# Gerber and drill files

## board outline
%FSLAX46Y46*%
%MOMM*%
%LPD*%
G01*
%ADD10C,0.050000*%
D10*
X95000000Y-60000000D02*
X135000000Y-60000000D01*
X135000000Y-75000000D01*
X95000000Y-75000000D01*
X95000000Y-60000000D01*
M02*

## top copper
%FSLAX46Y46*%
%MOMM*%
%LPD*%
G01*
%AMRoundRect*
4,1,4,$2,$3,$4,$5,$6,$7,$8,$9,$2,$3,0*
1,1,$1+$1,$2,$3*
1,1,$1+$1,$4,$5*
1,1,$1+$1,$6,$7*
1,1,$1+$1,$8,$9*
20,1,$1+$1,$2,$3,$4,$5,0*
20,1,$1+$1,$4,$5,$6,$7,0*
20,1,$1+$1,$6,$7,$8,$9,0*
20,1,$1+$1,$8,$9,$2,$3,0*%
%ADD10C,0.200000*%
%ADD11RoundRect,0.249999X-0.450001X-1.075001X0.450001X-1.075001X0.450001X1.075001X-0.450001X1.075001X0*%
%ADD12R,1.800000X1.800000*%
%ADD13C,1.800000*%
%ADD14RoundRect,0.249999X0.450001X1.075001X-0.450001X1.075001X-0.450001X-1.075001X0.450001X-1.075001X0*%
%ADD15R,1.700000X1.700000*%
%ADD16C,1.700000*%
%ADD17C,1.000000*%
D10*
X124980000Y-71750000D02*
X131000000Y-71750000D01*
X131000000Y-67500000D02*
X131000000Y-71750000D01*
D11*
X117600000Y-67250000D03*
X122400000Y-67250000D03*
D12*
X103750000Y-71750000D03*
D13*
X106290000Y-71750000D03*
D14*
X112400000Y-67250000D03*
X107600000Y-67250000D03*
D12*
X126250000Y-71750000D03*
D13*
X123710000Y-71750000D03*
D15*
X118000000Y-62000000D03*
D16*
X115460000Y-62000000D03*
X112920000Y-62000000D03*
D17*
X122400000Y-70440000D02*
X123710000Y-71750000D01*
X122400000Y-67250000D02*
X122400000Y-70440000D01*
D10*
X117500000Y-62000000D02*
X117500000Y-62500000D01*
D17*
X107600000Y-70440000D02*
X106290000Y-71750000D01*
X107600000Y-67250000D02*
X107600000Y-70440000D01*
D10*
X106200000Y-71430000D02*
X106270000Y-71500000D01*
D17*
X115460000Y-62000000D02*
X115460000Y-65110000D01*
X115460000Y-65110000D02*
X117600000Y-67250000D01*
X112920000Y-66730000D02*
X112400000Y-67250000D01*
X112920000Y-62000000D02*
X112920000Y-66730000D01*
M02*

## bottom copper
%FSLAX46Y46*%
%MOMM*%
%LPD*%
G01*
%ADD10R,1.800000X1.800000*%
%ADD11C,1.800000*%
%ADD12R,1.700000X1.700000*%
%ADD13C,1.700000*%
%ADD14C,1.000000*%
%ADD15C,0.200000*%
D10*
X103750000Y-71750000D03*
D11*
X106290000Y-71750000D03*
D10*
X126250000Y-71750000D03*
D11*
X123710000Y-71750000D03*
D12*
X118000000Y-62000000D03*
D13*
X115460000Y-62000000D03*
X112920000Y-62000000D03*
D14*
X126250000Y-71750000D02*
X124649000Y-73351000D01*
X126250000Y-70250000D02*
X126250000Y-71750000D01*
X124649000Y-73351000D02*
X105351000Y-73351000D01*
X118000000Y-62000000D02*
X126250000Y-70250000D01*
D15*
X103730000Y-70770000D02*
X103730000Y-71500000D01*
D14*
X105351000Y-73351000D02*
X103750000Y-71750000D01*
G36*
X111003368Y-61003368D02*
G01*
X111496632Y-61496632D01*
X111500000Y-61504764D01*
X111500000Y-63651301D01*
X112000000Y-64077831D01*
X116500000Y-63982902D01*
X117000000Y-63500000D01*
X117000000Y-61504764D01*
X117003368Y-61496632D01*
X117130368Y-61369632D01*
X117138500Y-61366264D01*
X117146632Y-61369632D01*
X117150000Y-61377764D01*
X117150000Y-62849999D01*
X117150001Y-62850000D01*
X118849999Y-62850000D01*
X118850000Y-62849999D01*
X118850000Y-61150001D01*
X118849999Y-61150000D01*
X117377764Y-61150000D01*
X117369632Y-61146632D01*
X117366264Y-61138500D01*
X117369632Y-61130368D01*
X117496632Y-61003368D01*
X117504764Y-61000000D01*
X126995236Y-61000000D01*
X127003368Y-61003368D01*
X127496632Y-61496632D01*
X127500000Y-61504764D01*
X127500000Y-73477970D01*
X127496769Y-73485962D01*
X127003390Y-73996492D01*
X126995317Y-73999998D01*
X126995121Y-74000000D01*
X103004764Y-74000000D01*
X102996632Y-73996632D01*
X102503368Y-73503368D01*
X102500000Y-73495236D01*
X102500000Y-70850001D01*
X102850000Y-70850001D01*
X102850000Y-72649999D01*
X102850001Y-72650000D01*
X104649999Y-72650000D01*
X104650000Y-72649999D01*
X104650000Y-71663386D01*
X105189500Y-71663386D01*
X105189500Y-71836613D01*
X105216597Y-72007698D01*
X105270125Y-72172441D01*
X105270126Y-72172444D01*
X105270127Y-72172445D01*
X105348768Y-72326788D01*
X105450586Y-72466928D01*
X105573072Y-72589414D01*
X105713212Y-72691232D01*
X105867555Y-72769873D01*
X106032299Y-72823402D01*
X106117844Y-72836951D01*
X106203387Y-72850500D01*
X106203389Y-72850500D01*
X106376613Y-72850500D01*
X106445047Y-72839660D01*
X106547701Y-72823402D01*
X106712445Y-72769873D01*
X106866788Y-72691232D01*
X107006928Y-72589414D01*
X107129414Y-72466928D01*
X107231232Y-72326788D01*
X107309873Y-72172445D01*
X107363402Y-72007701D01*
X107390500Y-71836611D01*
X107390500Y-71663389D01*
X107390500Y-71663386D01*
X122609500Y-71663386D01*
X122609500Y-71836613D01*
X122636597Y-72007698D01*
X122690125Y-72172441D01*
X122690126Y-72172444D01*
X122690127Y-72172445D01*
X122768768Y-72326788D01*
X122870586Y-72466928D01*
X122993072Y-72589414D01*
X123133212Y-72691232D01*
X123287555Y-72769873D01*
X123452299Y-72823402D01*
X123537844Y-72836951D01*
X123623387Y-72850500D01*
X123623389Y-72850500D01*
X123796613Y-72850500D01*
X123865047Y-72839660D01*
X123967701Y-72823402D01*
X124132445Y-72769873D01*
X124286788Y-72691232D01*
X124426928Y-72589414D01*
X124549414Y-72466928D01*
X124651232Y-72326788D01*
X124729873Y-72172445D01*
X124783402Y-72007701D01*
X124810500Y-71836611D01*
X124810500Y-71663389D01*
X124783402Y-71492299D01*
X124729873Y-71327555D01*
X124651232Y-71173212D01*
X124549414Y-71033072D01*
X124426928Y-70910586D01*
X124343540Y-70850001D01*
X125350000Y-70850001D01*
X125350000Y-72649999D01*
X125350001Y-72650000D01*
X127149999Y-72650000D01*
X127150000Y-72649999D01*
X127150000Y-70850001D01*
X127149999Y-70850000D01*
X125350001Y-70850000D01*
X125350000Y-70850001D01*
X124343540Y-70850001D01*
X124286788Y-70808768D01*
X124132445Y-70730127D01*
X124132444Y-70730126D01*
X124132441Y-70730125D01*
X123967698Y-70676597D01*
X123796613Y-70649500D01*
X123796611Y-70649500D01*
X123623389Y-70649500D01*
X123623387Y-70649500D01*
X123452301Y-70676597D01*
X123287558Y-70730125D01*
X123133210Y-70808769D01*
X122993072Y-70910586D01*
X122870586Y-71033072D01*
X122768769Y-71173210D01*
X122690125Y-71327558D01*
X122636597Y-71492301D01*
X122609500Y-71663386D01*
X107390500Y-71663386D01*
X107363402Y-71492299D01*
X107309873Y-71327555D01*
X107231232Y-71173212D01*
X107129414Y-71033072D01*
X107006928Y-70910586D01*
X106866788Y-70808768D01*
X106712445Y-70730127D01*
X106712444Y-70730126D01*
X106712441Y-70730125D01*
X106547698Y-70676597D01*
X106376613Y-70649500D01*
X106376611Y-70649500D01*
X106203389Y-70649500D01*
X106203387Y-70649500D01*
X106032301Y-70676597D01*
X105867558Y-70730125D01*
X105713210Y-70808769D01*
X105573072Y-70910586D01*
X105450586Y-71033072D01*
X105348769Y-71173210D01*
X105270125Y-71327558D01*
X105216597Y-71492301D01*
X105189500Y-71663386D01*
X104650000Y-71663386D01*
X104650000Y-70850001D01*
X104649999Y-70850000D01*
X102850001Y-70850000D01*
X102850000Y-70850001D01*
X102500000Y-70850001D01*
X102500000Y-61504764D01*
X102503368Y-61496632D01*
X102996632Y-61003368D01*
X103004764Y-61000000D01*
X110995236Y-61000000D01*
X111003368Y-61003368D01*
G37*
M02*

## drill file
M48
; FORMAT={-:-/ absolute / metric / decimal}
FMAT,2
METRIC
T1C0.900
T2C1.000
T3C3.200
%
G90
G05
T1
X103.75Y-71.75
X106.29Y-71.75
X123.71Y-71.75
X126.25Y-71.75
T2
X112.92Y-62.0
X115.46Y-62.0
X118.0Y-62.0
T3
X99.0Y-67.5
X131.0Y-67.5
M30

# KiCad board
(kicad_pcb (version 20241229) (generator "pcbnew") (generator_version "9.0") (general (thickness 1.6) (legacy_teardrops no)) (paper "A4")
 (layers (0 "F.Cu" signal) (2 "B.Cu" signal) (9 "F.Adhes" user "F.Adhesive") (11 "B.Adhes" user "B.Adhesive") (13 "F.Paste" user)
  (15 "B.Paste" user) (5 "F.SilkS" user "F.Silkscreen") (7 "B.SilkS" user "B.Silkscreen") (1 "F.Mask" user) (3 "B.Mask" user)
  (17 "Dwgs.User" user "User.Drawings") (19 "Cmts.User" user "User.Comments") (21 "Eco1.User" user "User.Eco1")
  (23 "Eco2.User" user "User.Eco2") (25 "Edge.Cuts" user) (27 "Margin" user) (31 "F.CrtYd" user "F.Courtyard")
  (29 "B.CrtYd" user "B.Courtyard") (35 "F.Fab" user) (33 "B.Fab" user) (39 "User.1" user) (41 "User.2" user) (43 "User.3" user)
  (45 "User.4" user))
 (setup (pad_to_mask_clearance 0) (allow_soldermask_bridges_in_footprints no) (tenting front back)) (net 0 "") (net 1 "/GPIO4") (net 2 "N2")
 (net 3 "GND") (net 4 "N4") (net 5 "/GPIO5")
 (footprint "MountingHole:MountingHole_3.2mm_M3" (layer "F.Cu") (at 131 67.5)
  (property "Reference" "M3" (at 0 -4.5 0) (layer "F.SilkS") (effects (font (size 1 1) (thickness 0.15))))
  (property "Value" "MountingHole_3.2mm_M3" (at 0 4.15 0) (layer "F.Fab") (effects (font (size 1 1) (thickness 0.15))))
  (pad "" np_thru_hole circle (at 0 0) (size 3.2 3.2) (drill 3.2) (layers "*.Cu" "*.Mask")))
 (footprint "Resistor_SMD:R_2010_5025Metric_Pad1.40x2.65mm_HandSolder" (layer "F.Cu") (at 120 67.25)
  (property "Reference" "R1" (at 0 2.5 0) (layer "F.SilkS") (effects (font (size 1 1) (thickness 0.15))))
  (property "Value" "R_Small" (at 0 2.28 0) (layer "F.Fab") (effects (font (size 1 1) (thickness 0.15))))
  (pad "1" smd roundrect (at -2.4 0) (size 1.4 2.65) (layers "F.Cu" "F.Mask" "F.Paste") (roundrect_rratio 0.178571) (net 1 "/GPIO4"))
  (pad "2" smd roundrect (at 2.4 0) (size 1.4 2.65) (layers "F.Cu" "F.Mask" "F.Paste") (roundrect_rratio 0.178571) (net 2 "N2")))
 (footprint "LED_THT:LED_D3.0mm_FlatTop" (layer "F.Cu") (at 103.75 71.75)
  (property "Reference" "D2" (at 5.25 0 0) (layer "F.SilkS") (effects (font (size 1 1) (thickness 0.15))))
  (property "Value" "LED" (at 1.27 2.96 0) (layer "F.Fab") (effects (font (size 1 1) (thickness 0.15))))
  (pad "1" thru_hole rect (at 0 0) (size 1.8 1.8) (drill 0.9) (layers "*.Cu" "*.Mask") (remove_unused_layers no) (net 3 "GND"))
  (pad "2" thru_hole circle (at 2.54 0) (size 1.8 1.8) (drill 0.9) (layers "*.Cu" "*.Mask") (remove_unused_layers no) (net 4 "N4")))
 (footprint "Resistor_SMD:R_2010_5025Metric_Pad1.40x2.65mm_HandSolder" (layer "F.Cu") (at 110 67.25 180)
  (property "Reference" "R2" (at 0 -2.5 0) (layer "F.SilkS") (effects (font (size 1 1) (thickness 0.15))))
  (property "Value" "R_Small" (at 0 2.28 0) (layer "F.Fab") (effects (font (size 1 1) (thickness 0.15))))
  (pad "1" smd roundrect (at -2.4 0 180) (size 1.4 2.65) (layers "F.Cu" "F.Mask" "F.Paste") (roundrect_rratio 0.178571) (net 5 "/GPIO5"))
  (pad "2" smd roundrect (at 2.4 0 180) (size 1.4 2.65) (layers "F.Cu" "F.Mask" "F.Paste") (roundrect_rratio 0.178571) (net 4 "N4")))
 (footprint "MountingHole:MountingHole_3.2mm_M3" (layer "F.Cu") (at 99 67.5)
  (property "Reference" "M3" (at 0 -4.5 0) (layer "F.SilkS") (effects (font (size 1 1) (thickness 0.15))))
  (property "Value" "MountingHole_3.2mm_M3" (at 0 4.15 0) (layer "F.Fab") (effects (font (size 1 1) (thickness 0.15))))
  (pad "" np_thru_hole circle (at 0 0) (size 3.2 3.2) (drill 3.2) (layers "*.Cu" "*.Mask")))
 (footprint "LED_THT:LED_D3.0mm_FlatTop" (layer "F.Cu") (at 126.25 71.75 180)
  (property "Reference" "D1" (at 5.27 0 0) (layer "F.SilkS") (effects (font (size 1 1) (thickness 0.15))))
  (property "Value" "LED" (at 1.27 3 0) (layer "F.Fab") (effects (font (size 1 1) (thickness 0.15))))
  (pad "1" thru_hole rect (at 0 0 180) (size 1.8 1.8) (drill 0.9) (layers "*.Cu" "*.Mask") (remove_unused_layers no) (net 3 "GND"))
  (pad "2" thru_hole circle (at 2.54 0 180) (size 1.8 1.8) (drill 0.9) (layers "*.Cu" "*.Mask") (remove_unused_layers no) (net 2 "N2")))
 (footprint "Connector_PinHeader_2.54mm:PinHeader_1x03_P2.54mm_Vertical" (layer "B.Cu") (at 118 62 90)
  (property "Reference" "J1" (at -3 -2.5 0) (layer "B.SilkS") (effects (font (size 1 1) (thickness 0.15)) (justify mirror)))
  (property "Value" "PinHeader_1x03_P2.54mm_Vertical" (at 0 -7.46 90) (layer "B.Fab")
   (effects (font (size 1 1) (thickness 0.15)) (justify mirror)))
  (pad "1" thru_hole rect (at 0 0 90) (size 1.7 1.7) (drill 1) (layers "*.Cu" "*.Mask") (remove_unused_layers no) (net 3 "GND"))
  (pad "2" thru_hole circle (at 0 -2.54 90) (size 1.7 1.7) (drill 1) (layers "*.Cu" "*.Mask") (remove_unused_layers no) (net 1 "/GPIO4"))
  (pad "3" thru_hole circle (at 0 -5.08 90) (size 1.7 1.7) (drill 1) (layers "*.Cu" "*.Mask") (remove_unused_layers no) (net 5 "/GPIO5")))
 (gr_line (start 124.98 71.75) (end 131 71.75) (stroke (width 0.2) (type default)) (layer "F.Cu") (net 3))
 (gr_line (start 131 67.5) (end 131 71.75) (stroke (width 0.2) (type default)) (layer "F.Cu") (net 3))
 (gr_rect (start 95 60) (end 135 75) (stroke (width 0.05) (type default)) (fill no) (layer "Edge.Cuts"))
 (segment (start 122.4 70.44) (end 123.71 71.75) (width 1) (layer "F.Cu") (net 2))
 (segment (start 122.4 67.25) (end 122.4 70.44) (width 1) (layer "F.Cu") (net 2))
 (segment (start 117.5 62) (end 117.5 62.5) (width 0.2) (layer "F.Cu") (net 3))
 (segment (start 126.25 71.75) (end 124.649 73.351) (width 1) (layer "B.Cu") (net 3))
 (segment (start 126.25 70.25) (end 126.25 71.75) (width 1) (layer "B.Cu") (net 3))
 (segment (start 124.649 73.351) (end 105.351 73.351) (width 1) (layer "B.Cu") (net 3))
 (segment (start 118 62) (end 126.25 70.25) (width 1) (layer "B.Cu") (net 3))
 (segment (start 103.73 70.77) (end 103.73 71.5) (width 0.2) (layer "B.Cu") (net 3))
 (segment (start 105.351 73.351) (end 103.75 71.75) (width 1) (layer "B.Cu") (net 3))
 (segment (start 107.6 70.44) (end 106.29 71.75) (width 1) (layer "F.Cu") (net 4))
 (segment (start 107.6 67.25) (end 107.6 70.44) (width 1) (layer "F.Cu") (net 4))
 (segment (start 106.2 71.43) (end 106.27 71.5) (width 0.2) (layer "F.Cu") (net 4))
 (segment (start 115.46 62) (end 115.46 65.11) (width 1) (layer "F.Cu") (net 1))
 (segment (start 115.46 65.11) (end 117.6 67.25) (width 1) (layer "F.Cu") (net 1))
 (segment (start 112.92 66.73) (end 112.4 67.25) (width 1) (layer "F.Cu") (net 5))
 (segment (start 112.92 62) (end 112.92 66.73) (width 1) (layer "F.Cu") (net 5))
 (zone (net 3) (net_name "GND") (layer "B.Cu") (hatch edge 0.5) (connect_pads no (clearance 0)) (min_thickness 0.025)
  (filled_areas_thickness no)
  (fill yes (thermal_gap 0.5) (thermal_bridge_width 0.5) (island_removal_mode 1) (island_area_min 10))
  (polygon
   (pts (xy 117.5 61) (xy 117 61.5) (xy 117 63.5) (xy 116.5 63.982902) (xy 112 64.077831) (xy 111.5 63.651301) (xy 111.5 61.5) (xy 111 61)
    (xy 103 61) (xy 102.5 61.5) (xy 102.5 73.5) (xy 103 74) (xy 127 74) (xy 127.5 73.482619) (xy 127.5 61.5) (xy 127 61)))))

